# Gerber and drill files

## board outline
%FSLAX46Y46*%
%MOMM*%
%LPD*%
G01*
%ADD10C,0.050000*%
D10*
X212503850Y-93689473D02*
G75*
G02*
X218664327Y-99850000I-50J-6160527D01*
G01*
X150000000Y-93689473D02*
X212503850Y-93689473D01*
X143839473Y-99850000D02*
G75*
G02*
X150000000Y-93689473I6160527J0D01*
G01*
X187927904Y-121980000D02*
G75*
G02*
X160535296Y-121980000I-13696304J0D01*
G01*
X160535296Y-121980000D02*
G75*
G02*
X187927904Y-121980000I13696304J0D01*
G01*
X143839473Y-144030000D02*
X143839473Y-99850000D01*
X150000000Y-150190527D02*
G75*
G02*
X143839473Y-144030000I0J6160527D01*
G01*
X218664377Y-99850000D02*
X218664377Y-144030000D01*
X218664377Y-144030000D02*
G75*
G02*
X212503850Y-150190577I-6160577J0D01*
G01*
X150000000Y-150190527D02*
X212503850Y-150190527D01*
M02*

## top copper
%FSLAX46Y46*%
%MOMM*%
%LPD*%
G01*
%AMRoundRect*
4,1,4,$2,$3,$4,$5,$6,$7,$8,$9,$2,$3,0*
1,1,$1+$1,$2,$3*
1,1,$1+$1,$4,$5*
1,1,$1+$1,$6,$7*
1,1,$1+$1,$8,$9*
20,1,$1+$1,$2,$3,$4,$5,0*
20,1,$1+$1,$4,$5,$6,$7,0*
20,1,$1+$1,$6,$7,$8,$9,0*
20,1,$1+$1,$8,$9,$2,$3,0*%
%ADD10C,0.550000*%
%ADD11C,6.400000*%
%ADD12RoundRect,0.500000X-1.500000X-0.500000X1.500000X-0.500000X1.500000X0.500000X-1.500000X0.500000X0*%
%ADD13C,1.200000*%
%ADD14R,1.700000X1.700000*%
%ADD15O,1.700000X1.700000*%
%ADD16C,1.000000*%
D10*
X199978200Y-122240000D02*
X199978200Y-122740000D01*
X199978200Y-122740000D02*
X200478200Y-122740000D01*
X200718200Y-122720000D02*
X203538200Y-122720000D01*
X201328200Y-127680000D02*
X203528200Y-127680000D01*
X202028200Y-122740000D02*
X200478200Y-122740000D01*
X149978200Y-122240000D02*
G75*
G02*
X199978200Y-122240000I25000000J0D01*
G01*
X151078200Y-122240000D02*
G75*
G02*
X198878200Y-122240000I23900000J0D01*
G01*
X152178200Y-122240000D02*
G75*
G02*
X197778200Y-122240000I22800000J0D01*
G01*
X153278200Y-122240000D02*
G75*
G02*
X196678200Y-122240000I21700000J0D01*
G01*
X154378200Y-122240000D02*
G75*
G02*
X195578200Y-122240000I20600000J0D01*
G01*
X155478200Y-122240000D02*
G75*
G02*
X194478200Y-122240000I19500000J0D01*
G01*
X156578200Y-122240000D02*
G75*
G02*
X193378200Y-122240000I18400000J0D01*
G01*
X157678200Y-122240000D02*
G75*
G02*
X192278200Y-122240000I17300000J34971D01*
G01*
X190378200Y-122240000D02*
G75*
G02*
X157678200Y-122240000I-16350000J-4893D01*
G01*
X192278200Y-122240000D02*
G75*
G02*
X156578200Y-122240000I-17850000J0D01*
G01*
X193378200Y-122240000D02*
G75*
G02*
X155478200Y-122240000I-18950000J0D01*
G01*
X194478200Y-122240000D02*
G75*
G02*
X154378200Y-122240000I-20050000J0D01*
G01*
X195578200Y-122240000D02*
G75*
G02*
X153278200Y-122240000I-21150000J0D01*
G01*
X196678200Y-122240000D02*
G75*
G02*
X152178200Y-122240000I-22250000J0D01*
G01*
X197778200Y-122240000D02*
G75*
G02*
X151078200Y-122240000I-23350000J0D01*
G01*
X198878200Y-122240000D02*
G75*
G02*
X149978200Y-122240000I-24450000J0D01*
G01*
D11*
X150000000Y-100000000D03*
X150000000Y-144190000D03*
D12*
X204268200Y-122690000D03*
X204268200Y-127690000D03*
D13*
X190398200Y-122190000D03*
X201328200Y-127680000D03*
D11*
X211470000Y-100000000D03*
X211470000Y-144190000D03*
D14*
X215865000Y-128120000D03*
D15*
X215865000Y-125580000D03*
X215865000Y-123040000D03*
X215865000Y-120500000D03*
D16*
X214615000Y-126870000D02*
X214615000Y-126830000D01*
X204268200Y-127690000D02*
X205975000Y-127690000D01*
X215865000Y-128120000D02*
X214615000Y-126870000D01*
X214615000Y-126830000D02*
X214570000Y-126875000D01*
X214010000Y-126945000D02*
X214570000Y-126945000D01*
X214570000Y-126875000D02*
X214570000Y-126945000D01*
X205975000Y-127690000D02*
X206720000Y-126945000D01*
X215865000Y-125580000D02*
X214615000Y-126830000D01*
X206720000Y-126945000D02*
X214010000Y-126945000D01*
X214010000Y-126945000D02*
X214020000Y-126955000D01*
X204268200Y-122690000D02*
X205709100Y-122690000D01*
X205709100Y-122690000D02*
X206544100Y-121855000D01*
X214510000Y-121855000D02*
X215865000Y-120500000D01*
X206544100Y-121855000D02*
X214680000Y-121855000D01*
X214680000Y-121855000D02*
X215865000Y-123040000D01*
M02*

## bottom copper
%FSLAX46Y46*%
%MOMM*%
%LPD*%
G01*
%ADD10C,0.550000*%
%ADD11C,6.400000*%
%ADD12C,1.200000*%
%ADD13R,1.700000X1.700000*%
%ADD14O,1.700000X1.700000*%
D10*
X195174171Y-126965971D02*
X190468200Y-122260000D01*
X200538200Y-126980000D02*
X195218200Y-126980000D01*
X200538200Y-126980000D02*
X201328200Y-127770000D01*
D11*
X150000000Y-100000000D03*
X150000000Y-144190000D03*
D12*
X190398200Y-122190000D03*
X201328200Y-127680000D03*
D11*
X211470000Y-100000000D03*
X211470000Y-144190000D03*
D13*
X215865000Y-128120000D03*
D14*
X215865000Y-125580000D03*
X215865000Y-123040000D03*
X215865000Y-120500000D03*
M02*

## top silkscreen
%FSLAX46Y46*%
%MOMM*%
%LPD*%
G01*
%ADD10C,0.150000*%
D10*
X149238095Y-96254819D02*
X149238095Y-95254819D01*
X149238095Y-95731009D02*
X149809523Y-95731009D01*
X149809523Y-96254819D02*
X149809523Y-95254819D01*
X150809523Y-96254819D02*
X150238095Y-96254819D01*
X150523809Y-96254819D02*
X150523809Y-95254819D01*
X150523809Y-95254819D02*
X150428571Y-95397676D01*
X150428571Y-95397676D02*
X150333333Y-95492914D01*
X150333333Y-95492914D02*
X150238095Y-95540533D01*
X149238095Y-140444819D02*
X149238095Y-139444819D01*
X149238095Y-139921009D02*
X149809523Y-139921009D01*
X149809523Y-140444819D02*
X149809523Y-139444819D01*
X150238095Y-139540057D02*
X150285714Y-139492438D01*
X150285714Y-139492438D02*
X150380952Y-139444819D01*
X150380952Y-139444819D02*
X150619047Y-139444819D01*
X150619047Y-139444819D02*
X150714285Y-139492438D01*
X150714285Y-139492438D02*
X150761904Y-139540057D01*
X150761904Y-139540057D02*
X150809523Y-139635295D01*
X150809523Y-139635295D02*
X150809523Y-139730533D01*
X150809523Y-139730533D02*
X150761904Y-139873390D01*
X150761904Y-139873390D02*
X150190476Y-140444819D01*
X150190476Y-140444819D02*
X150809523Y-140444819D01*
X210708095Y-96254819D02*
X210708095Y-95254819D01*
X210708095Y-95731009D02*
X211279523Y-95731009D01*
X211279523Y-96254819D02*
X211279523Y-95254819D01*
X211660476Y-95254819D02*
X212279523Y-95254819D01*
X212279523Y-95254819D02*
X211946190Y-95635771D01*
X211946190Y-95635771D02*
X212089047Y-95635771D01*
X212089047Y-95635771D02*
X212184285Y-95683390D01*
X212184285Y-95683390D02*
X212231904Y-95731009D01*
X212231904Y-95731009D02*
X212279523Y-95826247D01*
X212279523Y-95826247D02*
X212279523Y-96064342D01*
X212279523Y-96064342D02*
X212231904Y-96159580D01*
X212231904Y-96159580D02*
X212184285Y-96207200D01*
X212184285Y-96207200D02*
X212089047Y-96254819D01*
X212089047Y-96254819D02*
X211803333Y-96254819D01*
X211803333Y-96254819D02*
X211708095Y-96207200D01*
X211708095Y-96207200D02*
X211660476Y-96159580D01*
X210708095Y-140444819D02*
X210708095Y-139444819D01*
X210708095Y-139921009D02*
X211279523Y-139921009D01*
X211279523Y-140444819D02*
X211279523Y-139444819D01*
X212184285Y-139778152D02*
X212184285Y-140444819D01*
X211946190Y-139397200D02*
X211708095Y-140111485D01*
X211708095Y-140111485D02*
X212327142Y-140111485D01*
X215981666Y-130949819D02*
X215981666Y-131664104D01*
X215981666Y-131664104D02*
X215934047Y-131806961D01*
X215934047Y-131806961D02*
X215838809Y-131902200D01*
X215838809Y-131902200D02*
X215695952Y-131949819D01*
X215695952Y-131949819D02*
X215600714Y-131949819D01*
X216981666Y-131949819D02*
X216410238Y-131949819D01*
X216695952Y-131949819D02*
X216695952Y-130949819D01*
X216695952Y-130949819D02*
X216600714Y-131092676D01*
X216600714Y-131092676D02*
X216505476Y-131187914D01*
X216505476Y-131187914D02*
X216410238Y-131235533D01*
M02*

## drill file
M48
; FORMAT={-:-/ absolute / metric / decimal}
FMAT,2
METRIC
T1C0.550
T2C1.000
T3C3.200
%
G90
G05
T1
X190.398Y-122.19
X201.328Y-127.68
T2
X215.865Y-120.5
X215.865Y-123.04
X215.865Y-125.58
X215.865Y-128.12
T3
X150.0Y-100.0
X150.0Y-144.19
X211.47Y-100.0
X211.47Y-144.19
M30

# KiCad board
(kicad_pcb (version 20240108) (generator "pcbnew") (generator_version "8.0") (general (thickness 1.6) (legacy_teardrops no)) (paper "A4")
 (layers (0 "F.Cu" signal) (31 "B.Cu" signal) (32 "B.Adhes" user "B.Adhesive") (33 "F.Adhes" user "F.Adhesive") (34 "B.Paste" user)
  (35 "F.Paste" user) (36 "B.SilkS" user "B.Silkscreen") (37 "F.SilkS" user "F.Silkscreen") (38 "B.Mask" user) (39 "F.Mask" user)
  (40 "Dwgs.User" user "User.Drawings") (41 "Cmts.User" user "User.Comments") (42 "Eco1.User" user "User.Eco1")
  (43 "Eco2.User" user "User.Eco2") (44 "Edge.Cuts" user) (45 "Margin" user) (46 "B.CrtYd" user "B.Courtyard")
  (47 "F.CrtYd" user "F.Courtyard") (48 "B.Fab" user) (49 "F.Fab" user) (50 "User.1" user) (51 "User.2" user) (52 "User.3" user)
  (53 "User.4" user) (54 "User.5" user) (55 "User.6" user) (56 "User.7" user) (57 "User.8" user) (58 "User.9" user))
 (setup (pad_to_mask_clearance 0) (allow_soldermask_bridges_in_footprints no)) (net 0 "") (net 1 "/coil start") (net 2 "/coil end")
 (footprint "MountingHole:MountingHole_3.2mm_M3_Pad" (layer "F.Cu") (at 150 100)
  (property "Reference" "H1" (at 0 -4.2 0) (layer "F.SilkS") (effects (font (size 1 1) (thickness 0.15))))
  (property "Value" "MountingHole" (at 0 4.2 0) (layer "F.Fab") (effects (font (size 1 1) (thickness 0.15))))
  (pad "1" thru_hole circle (at 0 0) (size 6.4 6.4) (drill 3.2) (layers "*.Cu" "*.Mask") (remove_unused_layers no)))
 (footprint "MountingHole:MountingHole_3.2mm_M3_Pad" (layer "F.Cu") (at 150 144.19)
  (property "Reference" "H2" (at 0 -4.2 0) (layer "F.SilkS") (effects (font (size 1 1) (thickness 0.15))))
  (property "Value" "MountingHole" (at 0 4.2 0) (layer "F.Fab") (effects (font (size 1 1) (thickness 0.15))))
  (pad "1" thru_hole circle (at 0 0) (size 6.4 6.4) (drill 3.2) (layers "*.Cu" "*.Mask") (remove_unused_layers no)))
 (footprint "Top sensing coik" (layer "F.Cu") (at 174.4282 122.24)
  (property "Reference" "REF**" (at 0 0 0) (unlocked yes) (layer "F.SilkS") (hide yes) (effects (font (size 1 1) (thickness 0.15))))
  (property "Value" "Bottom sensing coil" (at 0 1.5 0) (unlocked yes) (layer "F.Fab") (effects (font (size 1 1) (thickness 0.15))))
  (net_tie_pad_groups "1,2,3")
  (fp_line (start 25.55 0) (end 25.55 0.5) (stroke (width 0.55) (type solid)) (layer "F.Cu"))
  (fp_line (start 25.55 0.5) (end 26.05 0.5) (stroke (width 0.55) (type solid)) (layer "F.Cu"))
  (fp_line (start 26.29 0.48) (end 29.11 0.48) (stroke (width 0.55) (type default)) (layer "F.Cu"))
  (fp_line (start 26.9 5.44) (end 29.1 5.44) (stroke (width 0.55) (type default)) (layer "F.Cu"))
  (fp_line (start 27.6 0.5) (end 26.05 0.5) (stroke (width 0.55) (type default)) (layer "F.Cu"))
  (fp_arc (start -24.45 0) (mid 0.55 -25) (end 25.55 0) (stroke (width 0.55) (type solid)) (layer "F.Cu"))
  (fp_arc (start -23.35 0) (mid 0.55 -23.9) (end 24.45 0) (stroke (width 0.55) (type solid)) (layer "F.Cu"))
  (fp_arc (start -22.25 0) (mid 0.55 -22.8) (end 23.35 0) (stroke (width 0.55) (type solid)) (layer "F.Cu"))
  (fp_arc (start -21.15 0) (mid 0.55 -21.7) (end 22.25 0) (stroke (width 0.55) (type solid)) (layer "F.Cu"))
  (fp_arc (start -20.05 0) (mid 0.55 -20.6) (end 21.15 0) (stroke (width 0.55) (type solid)) (layer "F.Cu"))
  (fp_arc (start -18.95 0) (mid 0.55 -19.5) (end 20.05 0) (stroke (width 0.55) (type solid)) (layer "F.Cu"))
  (fp_arc (start -17.85 0) (mid 0.55 -18.4) (end 18.95 0) (stroke (width 0.55) (type solid)) (layer "F.Cu"))
  (fp_arc (start -16.75 0) (mid 0.55 -17.335006) (end 17.85 0) (stroke (width 0.55) (type solid)) (layer "F.Cu"))
  (fp_arc (start 15.95 0) (mid -0.4 16.354894) (end -16.75 0) (stroke (width 0.55) (type solid)) (layer "F.Cu"))
  (fp_arc (start 17.85 0) (mid 0 17.85) (end -17.85 0) (stroke (width 0.55) (type solid)) (layer "F.Cu"))
  (fp_arc (start 18.95 0) (mid 0 18.95) (end -18.95 0) (stroke (width 0.55) (type solid)) (layer "F.Cu"))
  (fp_arc (start 20.05 0) (mid 0 20.05) (end -20.05 0) (stroke (width 0.55) (type solid)) (layer "F.Cu"))
  (fp_arc (start 21.15 0) (mid 0 21.15) (end -21.15 0) (stroke (width 0.55) (type solid)) (layer "F.Cu"))
  (fp_arc (start 22.25 0) (mid 0 22.25) (end -22.25 0) (stroke (width 0.55) (type solid)) (layer "F.Cu"))
  (fp_arc (start 23.35 0) (mid 0 23.35) (end -23.35 0) (stroke (width 0.55) (type solid)) (layer "F.Cu"))
  (fp_arc (start 24.45 0) (mid 0 24.45) (end -24.45 0) (stroke (width 0.55) (type solid)) (layer "F.Cu"))
  (fp_line (start 20.745971 4.725971) (end 16.04 0.02) (stroke (width 0.55) (type default)) (layer "B.Cu"))
  (fp_line (start 26.11 4.74) (end 20.79 4.74) (stroke (width 0.55) (type default)) (layer "B.Cu"))
  (fp_line (start 26.11 4.74) (end 26.9 5.53) (stroke (width 0.55) (type default)) (layer "B.Cu"))
  (pad "1" smd roundrect (at 29.84 0.45) (size 4 2) (layers "F.Cu") (roundrect_rratio 0.25) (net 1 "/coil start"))
  (pad "2" smd roundrect (at 29.84 5.45) (size 4 2) (layers "F.Cu") (roundrect_rratio 0.25) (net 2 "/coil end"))
  (pad "3" thru_hole circle (at 15.97 -0.05 90) (size 1.2 1.2) (drill 0.55) (layers "*.Cu" "*.Mask") (remove_unused_layers no))
  (pad "3" thru_hole circle (at 26.9 5.44 90) (size 1.2 1.2) (drill 0.55) (layers "*.Cu" "*.Mask") (remove_unused_layers no)))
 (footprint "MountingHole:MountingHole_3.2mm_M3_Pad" (layer "F.Cu") (at 211.47 100)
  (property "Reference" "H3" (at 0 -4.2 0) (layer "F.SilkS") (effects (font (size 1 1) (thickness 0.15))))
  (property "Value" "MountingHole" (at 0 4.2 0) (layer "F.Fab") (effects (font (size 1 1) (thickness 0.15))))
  (pad "1" thru_hole circle (at 0 0) (size 6.4 6.4) (drill 3.2) (layers "*.Cu" "*.Mask") (remove_unused_layers no)))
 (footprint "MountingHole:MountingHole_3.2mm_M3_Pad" (layer "F.Cu") (at 211.47 144.19)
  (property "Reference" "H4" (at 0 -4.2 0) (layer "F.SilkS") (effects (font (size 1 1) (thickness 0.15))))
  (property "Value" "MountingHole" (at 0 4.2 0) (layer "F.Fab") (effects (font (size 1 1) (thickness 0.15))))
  (pad "1" thru_hole circle (at 0 0) (size 6.4 6.4) (drill 3.2) (layers "*.Cu" "*.Mask") (remove_unused_layers no)))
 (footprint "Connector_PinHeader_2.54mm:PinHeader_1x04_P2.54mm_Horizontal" (layer "B.Cu") (at 215.865 128.12)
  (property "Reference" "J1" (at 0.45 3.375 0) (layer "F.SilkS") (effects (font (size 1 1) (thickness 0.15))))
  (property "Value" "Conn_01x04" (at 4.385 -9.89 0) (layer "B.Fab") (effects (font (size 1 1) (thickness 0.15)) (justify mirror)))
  (pad "1" thru_hole rect (at 0 0) (size 1.7 1.7) (drill 1) (layers "*.Cu" "*.Mask") (remove_unused_layers no) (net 2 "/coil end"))
  (pad "2" thru_hole oval (at 0 -2.54) (size 1.7 1.7) (drill 1) (layers "*.Cu" "*.Mask") (remove_unused_layers no) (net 2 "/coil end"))
  (pad "3" thru_hole oval (at 0 -5.08) (size 1.7 1.7) (drill 1) (layers "*.Cu" "*.Mask") (remove_unused_layers no) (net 1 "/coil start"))
  (pad "4" thru_hole oval (at 0 -7.62) (size 1.7 1.7) (drill 1) (layers "*.Cu" "*.Mask") (remove_unused_layers no) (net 1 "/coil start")))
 (gr_arc (start 212.50385 93.689473) (mid 216.86 95.49385) (end 218.664377 99.85) (stroke (width 0.05) (type default)) (layer "Edge.Cuts"))
 (gr_line (start 150 93.689473) (end 212.50385 93.689473) (stroke (width 0.05) (type default)) (layer "Edge.Cuts"))
 (gr_arc (start 143.839473 99.85) (mid 145.64385 95.49385) (end 150 93.689473) (stroke (width 0.05) (type default)) (layer "Edge.Cuts"))
 (gr_circle (center 174.2316 121.98) (end 186.47 115.830992) (stroke (width 0.05) (type default)) (fill none) (layer "Edge.Cuts"))
 (gr_line (start 143.839473 144.03) (end 143.839473 99.85) (stroke (width 0.05) (type default)) (layer "Edge.Cuts"))
 (gr_arc (start 150 150.190527) (mid 145.643849 148.38615) (end 143.839473 144.03) (stroke (width 0.05) (type default)) (layer "Edge.Cuts"))
 (gr_line (start 218.664377 99.85) (end 218.664377 144.03) (stroke (width 0.05) (type default)) (layer "Edge.Cuts"))
 (gr_arc (start 218.664377 144.03) (mid 216.86 148.38615) (end 212.50385 150.190527) (stroke (width 0.05) (type default))
  (layer "Edge.Cuts"))
 (gr_line (start 150 150.190527) (end 212.50385 150.190527) (stroke (width 0.05) (type default)) (layer "Edge.Cuts"))
 (segment (start 214.615 126.87) (end 214.615 126.83) (width 1) (layer "F.Cu") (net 2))
 (segment (start 204.2682 127.69) (end 205.975 127.69) (width 1) (layer "F.Cu") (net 2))
 (segment (start 215.865 128.12) (end 214.615 126.87) (width 1) (layer "F.Cu") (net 2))
 (segment (start 214.615 126.83) (end 214.57 126.875) (width 1) (layer "F.Cu") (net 2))
 (segment (start 214.01 126.945) (end 214.57 126.945) (width 1) (layer "F.Cu") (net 2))
 (segment (start 214.57 126.875) (end 214.57 126.945) (width 1) (layer "F.Cu") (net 2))
 (segment (start 205.975 127.69) (end 206.72 126.945) (width 1) (layer "F.Cu") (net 2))
 (segment (start 215.865 125.58) (end 214.615 126.83) (width 1) (layer "F.Cu") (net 2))
 (segment (start 206.72 126.945) (end 214.01 126.945) (width 1) (layer "F.Cu") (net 2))
 (segment (start 214.01 126.945) (end 214.02 126.955) (width 1) (layer "F.Cu") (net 2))
 (segment (start 204.2682 122.69) (end 205.7091 122.69) (width 1) (layer "F.Cu") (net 1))
 (segment (start 205.7091 122.69) (end 206.5441 121.855) (width 1) (layer "F.Cu") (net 1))
 (segment (start 214.51 121.855) (end 215.865 120.5) (width 1) (layer "F.Cu") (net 1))
 (segment (start 206.5441 121.855) (end 214.68 121.855) (width 1) (layer "F.Cu") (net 1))
 (segment (start 214.68 121.855) (end 215.865 123.04) (width 1) (layer "F.Cu") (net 1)))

